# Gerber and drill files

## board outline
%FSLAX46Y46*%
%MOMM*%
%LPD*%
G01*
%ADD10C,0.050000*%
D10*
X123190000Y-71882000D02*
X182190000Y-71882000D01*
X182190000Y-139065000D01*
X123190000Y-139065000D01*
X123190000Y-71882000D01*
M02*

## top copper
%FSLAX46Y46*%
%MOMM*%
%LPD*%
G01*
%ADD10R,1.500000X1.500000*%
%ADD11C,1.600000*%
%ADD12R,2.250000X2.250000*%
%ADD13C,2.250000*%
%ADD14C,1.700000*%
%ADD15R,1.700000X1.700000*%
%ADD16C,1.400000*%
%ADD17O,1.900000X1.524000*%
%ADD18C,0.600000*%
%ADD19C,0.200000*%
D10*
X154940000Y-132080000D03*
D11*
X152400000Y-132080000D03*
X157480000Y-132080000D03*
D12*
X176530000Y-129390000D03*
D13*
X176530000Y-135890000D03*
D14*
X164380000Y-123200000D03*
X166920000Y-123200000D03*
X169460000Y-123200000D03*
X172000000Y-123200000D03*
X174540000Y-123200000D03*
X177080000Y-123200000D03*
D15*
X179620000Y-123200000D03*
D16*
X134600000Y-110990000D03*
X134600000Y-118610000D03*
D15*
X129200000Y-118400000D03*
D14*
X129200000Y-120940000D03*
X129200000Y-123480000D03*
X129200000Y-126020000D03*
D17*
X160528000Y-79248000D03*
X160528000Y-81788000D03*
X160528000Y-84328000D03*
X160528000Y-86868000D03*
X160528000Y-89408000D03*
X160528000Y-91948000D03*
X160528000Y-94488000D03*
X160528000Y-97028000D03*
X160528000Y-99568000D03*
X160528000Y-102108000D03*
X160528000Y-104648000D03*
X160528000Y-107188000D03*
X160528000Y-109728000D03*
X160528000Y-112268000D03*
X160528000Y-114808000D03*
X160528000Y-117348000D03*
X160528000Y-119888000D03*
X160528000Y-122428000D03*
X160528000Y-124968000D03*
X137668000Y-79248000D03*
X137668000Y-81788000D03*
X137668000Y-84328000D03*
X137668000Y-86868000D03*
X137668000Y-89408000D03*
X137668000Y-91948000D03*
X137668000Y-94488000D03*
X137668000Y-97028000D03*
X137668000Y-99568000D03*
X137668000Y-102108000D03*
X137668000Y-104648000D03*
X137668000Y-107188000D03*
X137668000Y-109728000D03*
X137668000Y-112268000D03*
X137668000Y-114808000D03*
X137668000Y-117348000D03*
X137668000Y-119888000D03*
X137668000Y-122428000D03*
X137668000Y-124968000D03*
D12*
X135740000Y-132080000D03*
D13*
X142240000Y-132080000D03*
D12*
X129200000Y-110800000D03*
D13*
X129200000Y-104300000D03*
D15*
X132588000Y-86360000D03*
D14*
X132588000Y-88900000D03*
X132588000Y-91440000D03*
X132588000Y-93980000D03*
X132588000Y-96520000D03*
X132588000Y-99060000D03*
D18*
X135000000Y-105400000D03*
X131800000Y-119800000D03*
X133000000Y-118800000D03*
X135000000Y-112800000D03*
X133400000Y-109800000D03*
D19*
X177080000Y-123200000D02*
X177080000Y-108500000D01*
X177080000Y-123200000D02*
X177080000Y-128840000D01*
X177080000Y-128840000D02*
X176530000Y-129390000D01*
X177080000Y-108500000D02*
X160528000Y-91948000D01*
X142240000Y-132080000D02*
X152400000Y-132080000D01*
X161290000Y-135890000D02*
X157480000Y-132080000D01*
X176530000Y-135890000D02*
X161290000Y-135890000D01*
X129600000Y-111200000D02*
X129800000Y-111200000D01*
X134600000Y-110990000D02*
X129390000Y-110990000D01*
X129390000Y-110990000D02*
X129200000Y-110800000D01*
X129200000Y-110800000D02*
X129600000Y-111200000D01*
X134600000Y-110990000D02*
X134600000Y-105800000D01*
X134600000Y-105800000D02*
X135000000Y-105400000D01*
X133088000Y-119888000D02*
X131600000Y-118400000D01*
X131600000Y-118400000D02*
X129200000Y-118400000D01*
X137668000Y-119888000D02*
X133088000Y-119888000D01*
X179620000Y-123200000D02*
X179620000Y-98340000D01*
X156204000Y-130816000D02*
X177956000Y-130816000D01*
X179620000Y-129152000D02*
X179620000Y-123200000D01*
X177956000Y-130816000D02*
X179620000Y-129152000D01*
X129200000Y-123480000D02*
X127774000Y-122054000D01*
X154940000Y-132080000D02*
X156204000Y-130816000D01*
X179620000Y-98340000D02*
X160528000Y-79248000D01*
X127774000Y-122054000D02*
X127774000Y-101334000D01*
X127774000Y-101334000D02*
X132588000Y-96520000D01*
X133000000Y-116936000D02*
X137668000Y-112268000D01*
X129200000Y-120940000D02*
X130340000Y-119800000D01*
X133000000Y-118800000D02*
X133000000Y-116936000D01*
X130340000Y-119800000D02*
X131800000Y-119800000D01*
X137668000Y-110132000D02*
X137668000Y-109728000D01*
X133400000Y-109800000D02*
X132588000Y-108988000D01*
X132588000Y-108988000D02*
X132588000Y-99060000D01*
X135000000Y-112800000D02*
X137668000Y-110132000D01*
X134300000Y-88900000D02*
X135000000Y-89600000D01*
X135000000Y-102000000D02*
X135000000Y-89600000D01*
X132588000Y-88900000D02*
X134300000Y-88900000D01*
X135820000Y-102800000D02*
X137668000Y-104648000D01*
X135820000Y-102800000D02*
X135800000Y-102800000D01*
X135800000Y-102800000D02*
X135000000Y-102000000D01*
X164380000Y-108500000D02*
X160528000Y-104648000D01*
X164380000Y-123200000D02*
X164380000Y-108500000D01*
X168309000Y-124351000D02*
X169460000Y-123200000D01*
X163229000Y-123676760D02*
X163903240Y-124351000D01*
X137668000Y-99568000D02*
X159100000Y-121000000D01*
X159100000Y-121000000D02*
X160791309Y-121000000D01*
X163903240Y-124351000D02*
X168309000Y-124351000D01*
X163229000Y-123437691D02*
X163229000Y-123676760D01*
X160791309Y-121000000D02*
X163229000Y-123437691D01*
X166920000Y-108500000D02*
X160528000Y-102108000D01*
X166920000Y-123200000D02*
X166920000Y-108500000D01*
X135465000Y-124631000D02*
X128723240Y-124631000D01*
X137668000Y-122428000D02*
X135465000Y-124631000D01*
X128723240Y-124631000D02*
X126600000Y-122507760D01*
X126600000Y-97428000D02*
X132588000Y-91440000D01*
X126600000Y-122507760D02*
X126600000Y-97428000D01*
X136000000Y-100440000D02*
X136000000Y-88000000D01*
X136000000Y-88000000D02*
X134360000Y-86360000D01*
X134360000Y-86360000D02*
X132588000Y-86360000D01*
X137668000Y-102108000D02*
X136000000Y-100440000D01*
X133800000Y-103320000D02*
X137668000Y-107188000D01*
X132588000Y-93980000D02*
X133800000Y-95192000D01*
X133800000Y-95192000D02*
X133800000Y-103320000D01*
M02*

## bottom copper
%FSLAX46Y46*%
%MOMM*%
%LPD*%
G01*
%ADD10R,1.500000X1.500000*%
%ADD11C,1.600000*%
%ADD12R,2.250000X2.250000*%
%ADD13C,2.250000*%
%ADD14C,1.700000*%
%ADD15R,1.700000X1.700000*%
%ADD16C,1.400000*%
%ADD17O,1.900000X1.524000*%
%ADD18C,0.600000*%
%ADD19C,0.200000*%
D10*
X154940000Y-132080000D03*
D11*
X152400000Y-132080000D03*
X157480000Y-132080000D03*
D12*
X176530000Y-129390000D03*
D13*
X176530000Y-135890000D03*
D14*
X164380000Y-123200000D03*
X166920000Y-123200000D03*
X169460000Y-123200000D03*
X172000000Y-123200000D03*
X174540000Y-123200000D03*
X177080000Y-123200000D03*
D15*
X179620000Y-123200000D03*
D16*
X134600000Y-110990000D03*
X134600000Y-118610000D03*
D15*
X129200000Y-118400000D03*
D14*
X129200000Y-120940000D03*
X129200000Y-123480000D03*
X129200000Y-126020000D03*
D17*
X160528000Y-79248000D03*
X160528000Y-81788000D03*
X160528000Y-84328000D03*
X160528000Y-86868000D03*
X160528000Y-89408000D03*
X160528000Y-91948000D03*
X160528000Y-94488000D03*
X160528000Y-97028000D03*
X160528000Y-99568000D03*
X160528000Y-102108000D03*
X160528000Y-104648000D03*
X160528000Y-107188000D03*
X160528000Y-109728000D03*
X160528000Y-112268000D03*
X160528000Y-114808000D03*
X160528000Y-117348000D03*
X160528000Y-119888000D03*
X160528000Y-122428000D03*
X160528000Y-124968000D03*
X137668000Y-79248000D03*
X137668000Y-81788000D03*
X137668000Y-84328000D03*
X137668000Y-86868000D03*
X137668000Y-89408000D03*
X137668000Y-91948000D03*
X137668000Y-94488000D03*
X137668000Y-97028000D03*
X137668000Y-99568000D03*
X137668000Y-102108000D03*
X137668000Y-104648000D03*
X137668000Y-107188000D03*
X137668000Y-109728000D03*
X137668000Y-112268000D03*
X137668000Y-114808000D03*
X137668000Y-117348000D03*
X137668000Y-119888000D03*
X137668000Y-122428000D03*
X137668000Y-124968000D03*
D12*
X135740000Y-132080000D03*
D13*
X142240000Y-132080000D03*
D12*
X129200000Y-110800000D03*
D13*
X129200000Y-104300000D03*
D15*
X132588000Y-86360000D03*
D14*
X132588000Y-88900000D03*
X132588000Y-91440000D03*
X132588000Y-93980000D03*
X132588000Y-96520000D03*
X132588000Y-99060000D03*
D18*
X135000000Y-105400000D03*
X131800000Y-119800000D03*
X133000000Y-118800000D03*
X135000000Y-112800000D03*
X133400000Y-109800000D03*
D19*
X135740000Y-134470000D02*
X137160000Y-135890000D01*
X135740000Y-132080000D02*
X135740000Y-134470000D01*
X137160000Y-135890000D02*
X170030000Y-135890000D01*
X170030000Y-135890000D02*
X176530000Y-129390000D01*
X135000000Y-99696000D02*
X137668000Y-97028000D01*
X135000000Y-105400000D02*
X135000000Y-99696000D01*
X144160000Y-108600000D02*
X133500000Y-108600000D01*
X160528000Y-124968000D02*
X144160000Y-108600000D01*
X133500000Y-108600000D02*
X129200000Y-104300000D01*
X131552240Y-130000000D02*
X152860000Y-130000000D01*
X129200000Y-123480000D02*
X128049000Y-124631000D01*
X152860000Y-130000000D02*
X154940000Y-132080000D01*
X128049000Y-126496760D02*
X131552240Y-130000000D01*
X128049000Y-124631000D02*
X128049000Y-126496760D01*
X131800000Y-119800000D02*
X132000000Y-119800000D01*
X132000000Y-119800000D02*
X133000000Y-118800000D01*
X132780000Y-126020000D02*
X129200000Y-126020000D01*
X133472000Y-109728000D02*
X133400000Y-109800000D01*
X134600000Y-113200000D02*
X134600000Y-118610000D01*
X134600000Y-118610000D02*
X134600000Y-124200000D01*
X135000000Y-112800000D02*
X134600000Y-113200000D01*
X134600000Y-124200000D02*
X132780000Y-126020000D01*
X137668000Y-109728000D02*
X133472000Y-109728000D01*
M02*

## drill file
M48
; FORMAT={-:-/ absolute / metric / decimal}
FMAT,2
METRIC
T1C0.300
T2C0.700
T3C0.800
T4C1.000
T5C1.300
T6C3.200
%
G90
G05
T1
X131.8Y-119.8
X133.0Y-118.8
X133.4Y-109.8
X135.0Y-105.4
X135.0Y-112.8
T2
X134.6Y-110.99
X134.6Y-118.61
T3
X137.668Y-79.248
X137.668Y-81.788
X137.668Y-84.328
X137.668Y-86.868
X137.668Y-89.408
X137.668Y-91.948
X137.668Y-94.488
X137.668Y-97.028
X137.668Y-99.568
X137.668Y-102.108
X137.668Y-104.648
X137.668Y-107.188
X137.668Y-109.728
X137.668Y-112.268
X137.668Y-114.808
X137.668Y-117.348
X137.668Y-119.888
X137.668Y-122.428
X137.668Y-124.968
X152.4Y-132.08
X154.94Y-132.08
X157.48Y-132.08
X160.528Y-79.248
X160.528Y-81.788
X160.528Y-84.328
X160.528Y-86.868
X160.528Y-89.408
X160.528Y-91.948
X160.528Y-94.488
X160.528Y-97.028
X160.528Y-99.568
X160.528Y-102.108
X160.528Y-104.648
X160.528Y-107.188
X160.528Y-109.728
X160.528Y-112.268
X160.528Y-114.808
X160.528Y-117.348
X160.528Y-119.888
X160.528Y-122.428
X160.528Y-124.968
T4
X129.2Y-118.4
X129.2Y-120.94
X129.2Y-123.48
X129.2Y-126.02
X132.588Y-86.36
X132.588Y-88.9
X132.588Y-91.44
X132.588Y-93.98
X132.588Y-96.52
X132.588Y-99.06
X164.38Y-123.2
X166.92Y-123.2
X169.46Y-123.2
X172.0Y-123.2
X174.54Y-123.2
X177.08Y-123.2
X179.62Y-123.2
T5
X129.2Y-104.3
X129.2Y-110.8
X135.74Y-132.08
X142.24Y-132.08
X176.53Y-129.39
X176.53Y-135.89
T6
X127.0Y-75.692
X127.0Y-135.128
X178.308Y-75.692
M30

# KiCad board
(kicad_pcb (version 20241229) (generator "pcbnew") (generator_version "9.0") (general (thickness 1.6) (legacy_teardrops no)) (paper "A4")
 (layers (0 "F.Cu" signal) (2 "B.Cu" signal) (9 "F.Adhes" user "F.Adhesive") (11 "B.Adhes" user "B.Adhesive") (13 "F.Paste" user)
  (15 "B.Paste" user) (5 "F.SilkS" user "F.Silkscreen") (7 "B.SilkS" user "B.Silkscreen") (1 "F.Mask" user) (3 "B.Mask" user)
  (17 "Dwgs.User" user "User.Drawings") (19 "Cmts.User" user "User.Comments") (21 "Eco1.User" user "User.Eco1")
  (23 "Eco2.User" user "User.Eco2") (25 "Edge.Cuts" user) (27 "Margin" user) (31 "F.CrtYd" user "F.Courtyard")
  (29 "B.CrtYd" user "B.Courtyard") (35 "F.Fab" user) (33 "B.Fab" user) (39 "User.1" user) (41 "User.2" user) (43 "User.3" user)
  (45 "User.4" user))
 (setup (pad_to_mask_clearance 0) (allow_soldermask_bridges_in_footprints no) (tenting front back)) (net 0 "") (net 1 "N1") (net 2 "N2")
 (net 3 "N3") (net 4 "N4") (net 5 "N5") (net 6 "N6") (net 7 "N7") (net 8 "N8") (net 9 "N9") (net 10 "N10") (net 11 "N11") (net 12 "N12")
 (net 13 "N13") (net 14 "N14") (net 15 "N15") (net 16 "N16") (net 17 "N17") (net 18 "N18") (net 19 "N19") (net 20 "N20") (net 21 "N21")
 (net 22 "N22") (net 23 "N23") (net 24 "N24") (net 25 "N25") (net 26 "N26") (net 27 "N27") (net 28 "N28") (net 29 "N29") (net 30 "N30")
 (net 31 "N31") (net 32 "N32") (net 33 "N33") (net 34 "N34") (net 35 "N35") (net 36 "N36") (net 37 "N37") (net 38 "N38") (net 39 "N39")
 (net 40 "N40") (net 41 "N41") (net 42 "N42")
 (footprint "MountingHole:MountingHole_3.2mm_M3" (layer "F.Cu") (at 178.308 75.692)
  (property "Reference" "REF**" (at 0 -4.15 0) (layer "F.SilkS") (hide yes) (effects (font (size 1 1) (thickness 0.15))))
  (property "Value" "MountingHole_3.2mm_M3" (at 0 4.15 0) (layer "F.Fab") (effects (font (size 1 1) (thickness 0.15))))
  (pad "" np_thru_hole circle (at 0 0) (size 3.2 3.2) (drill 3.2) (layers "*.Cu" "*.Mask")))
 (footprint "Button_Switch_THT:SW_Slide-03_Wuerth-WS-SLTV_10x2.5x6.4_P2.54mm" (layer "F.Cu") (at 154.94 132.08)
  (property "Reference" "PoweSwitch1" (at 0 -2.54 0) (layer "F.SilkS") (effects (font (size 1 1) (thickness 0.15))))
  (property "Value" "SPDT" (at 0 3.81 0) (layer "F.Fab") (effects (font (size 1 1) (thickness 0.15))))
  (pad "1" thru_hole rect (at 0 0) (size 1.5 1.5) (drill 0.8) (layers "*.Cu" "*.Mask") (remove_unused_layers no) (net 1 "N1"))
  (pad "2" thru_hole circle (at -2.54 0) (size 1.6 1.6) (drill 0.8) (layers "*.Cu" "*.Mask") (remove_unused_layers no) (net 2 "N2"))
  (pad "3" thru_hole circle (at 2.54 0) (size 1.6 1.6) (drill 0.8) (layers "*.Cu" "*.Mask") (remove_unused_layers no) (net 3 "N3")))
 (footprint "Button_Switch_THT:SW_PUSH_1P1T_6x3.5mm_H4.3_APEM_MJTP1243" (layer "F.Cu") (at 176.53 129.39 -90)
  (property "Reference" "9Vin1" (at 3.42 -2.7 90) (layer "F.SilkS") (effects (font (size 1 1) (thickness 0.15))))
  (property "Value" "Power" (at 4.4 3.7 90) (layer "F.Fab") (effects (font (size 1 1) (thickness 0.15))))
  (pad "1" thru_hole rect (at 0 0) (size 2.25 2.25) (drill 1.3) (layers "*.Cu" "*.Mask") (remove_unused_layers no) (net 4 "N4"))
  (pad "2" thru_hole circle (at 6.5 0) (size 2.25 2.25) (drill 1.3) (layers "*.Cu" "*.Mask") (remove_unused_layers no) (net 3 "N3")))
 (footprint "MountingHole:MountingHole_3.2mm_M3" (layer "F.Cu") (at 127 135.128)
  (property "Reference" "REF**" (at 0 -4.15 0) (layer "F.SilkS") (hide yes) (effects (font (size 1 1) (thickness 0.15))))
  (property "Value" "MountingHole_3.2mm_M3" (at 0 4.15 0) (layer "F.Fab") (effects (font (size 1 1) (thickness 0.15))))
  (pad "" np_thru_hole circle (at 0 0) (size 3.2 3.2) (drill 3.2) (layers "*.Cu" "*.Mask")))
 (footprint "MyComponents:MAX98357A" (layer "F.Cu") (at 164.38 123.2 90)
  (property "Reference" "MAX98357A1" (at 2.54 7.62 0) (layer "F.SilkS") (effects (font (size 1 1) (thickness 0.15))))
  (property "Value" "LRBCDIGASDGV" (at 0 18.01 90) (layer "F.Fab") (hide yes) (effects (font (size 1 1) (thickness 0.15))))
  (pad "1" thru_hole circle (at 0 0 270) (size 1.7 1.7) (drill 1) (layers "*.Cu" "*.Mask") (remove_unused_layers no) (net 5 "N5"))
  (pad "2" thru_hole circle (at 0 2.54 270) (size 1.7 1.7) (drill 1) (layers "*.Cu" "*.Mask") (remove_unused_layers no) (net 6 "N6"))
  (pad "3" thru_hole circle (at 0 5.08 270) (size 1.7 1.7) (drill 1) (layers "*.Cu" "*.Mask") (remove_unused_layers no) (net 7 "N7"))
  (pad "4" thru_hole circle (at 0 7.62 270) (size 1.7 1.7) (drill 1) (layers "*.Cu" "*.Mask") (remove_unused_layers no) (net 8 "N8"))
  (pad "5" thru_hole circle (at 0 10.16 270) (size 1.7 1.7) (drill 1) (layers "*.Cu" "*.Mask") (remove_unused_layers no) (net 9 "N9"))
  (pad "6" thru_hole circle (at 0 12.7 270) (size 1.7 1.7) (drill 1) (layers "*.Cu" "*.Mask") (remove_unused_layers no) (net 4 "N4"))
  (pad "7" thru_hole rect (at 0 15.24 270) (size 1.7 1.7) (drill 1) (layers "*.Cu" "*.Mask") (remove_unused_layers no) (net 1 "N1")))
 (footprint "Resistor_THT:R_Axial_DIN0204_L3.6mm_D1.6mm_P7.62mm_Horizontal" (layer "F.Cu") (at 134.6 110.99 -90)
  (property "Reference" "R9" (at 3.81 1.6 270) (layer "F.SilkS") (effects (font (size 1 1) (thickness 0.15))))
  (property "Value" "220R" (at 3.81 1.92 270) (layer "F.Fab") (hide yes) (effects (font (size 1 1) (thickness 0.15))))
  (pad "1" thru_hole circle (at 0 0 270) (size 1.4 1.4) (drill 0.7) (layers "*.Cu" "*.Mask") (remove_unused_layers no) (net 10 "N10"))
  (pad "2" thru_hole circle (at 7.62 0 270) (size 1.4 1.4) (drill 0.7) (layers "*.Cu" "*.Mask") (remove_unused_layers no) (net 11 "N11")))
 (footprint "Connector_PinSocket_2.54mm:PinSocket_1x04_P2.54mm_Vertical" (layer "F.Cu") (at 129.2 118.4)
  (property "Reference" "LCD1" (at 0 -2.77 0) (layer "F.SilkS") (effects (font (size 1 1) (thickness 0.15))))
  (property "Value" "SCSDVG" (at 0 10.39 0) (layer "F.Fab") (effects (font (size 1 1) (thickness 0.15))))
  (pad "1" thru_hole rect (at 0 0) (size 1.7 1.7) (drill 1) (layers "*.Cu" "*.Mask") (remove_unused_layers no) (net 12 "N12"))
  (pad "2" thru_hole circle (at 0 2.54) (size 1.7 1.7) (drill 1) (layers "*.Cu" "*.Mask") (remove_unused_layers no) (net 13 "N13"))
  (pad "3" thru_hole circle (at 0 5.08) (size 1.7 1.7) (drill 1) (layers "*.Cu" "*.Mask") (remove_unused_layers no) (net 1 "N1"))
  (pad "4" thru_hole circle (at 0 7.62) (size 1.7 1.7) (drill 1) (layers "*.Cu" "*.Mask") (remove_unused_layers no) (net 11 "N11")))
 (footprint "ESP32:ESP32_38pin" (layer "F.Cu") (at 148.984183 102.273111 180)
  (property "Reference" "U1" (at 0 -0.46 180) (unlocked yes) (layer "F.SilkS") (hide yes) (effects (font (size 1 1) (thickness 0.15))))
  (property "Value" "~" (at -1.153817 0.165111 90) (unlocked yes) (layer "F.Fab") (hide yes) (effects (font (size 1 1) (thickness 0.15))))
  (pad "1" thru_hole oval (at -11.543817 23.025111 90) (size 1.524 1.9) (drill 0.8) (layers "*.Cu" "*.Mask") (remove_unused_layers no)
   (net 1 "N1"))
  (pad "2" thru_hole oval (at -11.543817 20.485111 90) (size 1.524 1.9) (drill 0.8) (layers "*.Cu" "*.Mask") (remove_unused_layers no)
   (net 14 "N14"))
  (pad "3" thru_hole oval (at -11.543817 17.945111 90) (size 1.524 1.9) (drill 0.8) (layers "*.Cu" "*.Mask") (remove_unused_layers no)
   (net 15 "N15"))
  (pad "4" thru_hole oval (at -11.543817 15.405111 90) (size 1.524 1.9) (drill 0.8) (layers "*.Cu" "*.Mask") (remove_unused_layers no)
   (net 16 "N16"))
  (pad "5" thru_hole oval (at -11.543817 12.865111 90) (size 1.524 1.9) (drill 0.8) (layers "*.Cu" "*.Mask") (remove_unused_layers no)
   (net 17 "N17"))
  (pad "6" thru_hole oval (at -11.543817 10.325111 90) (size 1.524 1.9) (drill 0.8) (layers "*.Cu" "*.Mask") (remove_unused_layers no)
   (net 4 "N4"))
  (pad "7" thru_hole oval (at -11.543817 7.785111 90) (size 1.524 1.9) (drill 0.8) (layers "*.Cu" "*.Mask") (remove_unused_layers no)
   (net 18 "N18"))
  (pad "8" thru_hole oval (at -11.543817 5.245111 90) (size 1.524 1.9) (drill 0.8) (layers "*.Cu" "*.Mask") (remove_unused_layers no)
   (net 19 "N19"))
  (pad "9" thru_hole oval (at -11.543817 2.705111 90) (size 1.524 1.9) (drill 0.8) (layers "*.Cu" "*.Mask") (remove_unused_layers no)
   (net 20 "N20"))
  (pad "10" thru_hole oval (at -11.543817 0.165111 90) (size 1.524 1.9) (drill 0.8) (layers "*.Cu" "*.Mask") (remove_unused_layers no)
   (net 6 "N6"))
  (pad "11" thru_hole oval (at -11.543817 -2.374889 90) (size 1.524 1.9) (drill 0.8) (layers "*.Cu" "*.Mask") (remove_unused_layers no)
   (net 5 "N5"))
  (pad "12" thru_hole oval (at -11.543817 -4.914889 90) (size 1.524 1.9) (drill 0.8) (layers "*.Cu" "*.Mask") (remove_unused_layers no)
   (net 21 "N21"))
  (pad "13" thru_hole oval (at -11.543817 -7.454889 90) (size 1.524 1.9) (drill 0.8) (layers "*.Cu" "*.Mask") (remove_unused_layers no)
   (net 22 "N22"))
  (pad "14" thru_hole oval (at -11.543817 -9.994889 90) (size 1.524 1.9) (drill 0.8) (layers "*.Cu" "*.Mask") (remove_unused_layers no)
   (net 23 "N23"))
  (pad "15" thru_hole oval (at -11.543817 -12.534889 90) (size 1.524 1.9) (drill 0.8) (layers "*.Cu" "*.Mask") (remove_unused_layers no)
   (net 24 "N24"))
  (pad "16" thru_hole oval (at -11.543817 -15.074889 90) (size 1.524 1.9) (drill 0.8) (layers "*.Cu" "*.Mask") (remove_unused_layers no)
   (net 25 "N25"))
  (pad "17" thru_hole oval (at -11.543817 -17.614889 90) (size 1.524 1.9) (drill 0.8) (layers "*.Cu" "*.Mask") (remove_unused_layers no)
   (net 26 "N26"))
  (pad "18" thru_hole oval (at -11.543817 -20.154889 90) (size 1.524 1.9) (drill 0.8) (layers "*.Cu" "*.Mask") (remove_unused_layers no)
   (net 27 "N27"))
  (pad "19" thru_hole oval (at -11.543817 -22.694889 90) (size 1.524 1.9) (drill 0.8) (layers "*.Cu" "*.Mask") (remove_unused_layers no)
   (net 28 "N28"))
  (pad "20" thru_hole oval (at 11.316183 23.025111 90) (size 1.524 1.9) (drill 0.8) (layers "*.Cu" "*.Mask") (remove_unused_layers no)
   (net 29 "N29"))
  (pad "21" thru_hole oval (at 11.316183 20.485111 90) (size 1.524 1.9) (drill 0.8) (layers "*.Cu" "*.Mask") (remove_unused_layers no)
   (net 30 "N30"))
  (pad "22" thru_hole oval (at 11.316183 17.945111 90) (size 1.524 1.9) (drill 0.8) (layers "*.Cu" "*.Mask") (remove_unused_layers no)
   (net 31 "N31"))
  (pad "23" thru_hole oval (at 11.316183 15.405111 90) (size 1.524 1.9) (drill 0.8) (layers "*.Cu" "*.Mask") (remove_unused_layers no)
   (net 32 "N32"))
  (pad "24" thru_hole oval (at 11.316183 12.865111 90) (size 1.524 1.9) (drill 0.8) (layers "*.Cu" "*.Mask") (remove_unused_layers no)
   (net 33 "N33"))
  (pad "25" thru_hole oval (at 11.316183 10.325111 90) (size 1.524 1.9) (drill 0.8) (layers "*.Cu" "*.Mask") (remove_unused_layers no)
   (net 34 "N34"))
  (pad "26" thru_hole oval (at 11.316183 7.785111 90) (size 1.524 1.9) (drill 0.8) (layers "*.Cu" "*.Mask") (remove_unused_layers no)
   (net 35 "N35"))
  (pad "27" thru_hole oval (at 11.316183 5.245111 90) (size 1.524 1.9) (drill 0.8) (layers "*.Cu" "*.Mask") (remove_unused_layers no)
   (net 10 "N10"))
  (pad "28" thru_hole oval (at 11.316183 2.705111 90) (size 1.524 1.9) (drill 0.8) (layers "*.Cu" "*.Mask") (remove_unused_layers no)
   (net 7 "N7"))
  (pad "29" thru_hole oval (at 11.316183 0.165111 90) (size 1.524 1.9) (drill 0.8) (layers "*.Cu" "*.Mask") (remove_unused_layers no)
   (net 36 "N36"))
  (pad "30" thru_hole oval (at 11.316183 -2.374889 90) (size 1.524 1.9) (drill 0.8) (layers "*.Cu" "*.Mask") (remove_unused_layers no)
   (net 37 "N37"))
  (pad "31" thru_hole oval (at 11.316183 -4.914889 90) (size 1.524 1.9) (drill 0.8) (layers "*.Cu" "*.Mask") (remove_unused_layers no)
   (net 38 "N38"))
  (pad "32" thru_hole oval (at 11.316183 -7.454889 90) (size 1.524 1.9) (drill 0.8) (layers "*.Cu" "*.Mask") (remove_unused_layers no)
   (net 11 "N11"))
  (pad "33" thru_hole oval (at 11.316183 -9.994889 90) (size 1.524 1.9) (drill 0.8) (layers "*.Cu" "*.Mask") (remove_unused_layers no)
   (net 13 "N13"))
  (pad "34" thru_hole oval (at 11.316183 -12.534889 90) (size 1.524 1.9) (drill 0.8) (layers "*.Cu" "*.Mask") (remove_unused_layers no)
   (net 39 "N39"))
  (pad "35" thru_hole oval (at 11.316183 -15.074889 90) (size 1.524 1.9) (drill 0.8) (layers "*.Cu" "*.Mask") (remove_unused_layers no)
   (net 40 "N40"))
  (pad "36" thru_hole oval (at 11.316183 -17.614889 90) (size 1.524 1.9) (drill 0.8) (layers "*.Cu" "*.Mask") (remove_unused_layers no)
   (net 12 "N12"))
  (pad "37" thru_hole oval (at 11.316183 -20.154889 90) (size 1.524 1.9) (drill 0.8) (layers "*.Cu" "*.Mask") (remove_unused_layers no)
   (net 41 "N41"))
  (pad "38" thru_hole oval (at 11.316183 -22.694889 90) (size 1.524 1.9) (drill 0.8) (layers "*.Cu" "*.Mask") (remove_unused_layers no)
   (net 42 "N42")))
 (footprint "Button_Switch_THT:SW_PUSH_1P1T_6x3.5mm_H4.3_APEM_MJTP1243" (layer "F.Cu") (at 135.74 132.08)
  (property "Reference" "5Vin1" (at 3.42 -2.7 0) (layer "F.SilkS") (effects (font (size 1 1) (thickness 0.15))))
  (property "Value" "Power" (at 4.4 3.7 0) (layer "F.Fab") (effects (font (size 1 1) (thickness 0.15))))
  (pad "1" thru_hole rect (at 0 0 90) (size 2.25 2.25) (drill 1.3) (layers "*.Cu" "*.Mask") (remove_unused_layers no) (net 4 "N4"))
  (pad "2" thru_hole circle (at 6.5 0 90) (size 2.25 2.25) (drill 1.3) (layers "*.Cu" "*.Mask") (remove_unused_layers no) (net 2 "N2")))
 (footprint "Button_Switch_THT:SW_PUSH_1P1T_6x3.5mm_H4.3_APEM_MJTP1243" (layer "F.Cu") (at 129.2 110.8 90)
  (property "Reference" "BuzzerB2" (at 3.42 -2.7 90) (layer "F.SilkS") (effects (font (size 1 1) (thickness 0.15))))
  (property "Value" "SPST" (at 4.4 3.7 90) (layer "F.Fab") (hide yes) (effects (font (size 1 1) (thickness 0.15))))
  (pad "1" thru_hole rect (at 0 0 180) (size 2.25 2.25) (drill 1.3) (layers "*.Cu" "*.Mask") (remove_unused_layers no) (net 10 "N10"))
  (pad "2" thru_hole circle (at 6.5 0 180) (size 2.25 2.25) (drill 1.3) (layers "*.Cu" "*.Mask") (remove_unused_layers no) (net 28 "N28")))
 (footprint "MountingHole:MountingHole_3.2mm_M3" (layer "F.Cu") (at 127 75.692)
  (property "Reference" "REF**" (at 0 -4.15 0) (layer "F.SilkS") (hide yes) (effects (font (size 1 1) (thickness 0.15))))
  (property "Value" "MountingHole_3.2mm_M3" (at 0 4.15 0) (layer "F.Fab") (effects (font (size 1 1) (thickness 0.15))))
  (pad "" np_thru_hole circle (at 0 0) (size 3.2 3.2) (drill 3.2) (layers "*.Cu" "*.Mask")))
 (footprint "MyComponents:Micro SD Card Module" (layer "B.Cu") (at 132.588 86.435 180)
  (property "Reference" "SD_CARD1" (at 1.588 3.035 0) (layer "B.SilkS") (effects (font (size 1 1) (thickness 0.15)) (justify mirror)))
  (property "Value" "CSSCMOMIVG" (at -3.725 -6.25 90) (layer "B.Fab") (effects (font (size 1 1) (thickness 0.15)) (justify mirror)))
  (pad "1" thru_hole rect (at 0 0.075 180) (size 1.7 1.7) (drill 1) (layers "*.Cu" "*.Mask") (remove_unused_layers no) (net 36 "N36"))
  (pad "2" thru_hole circle (at 0 -2.465 180) (size 1.7 1.7) (drill 1) (layers "*.Cu" "*.Mask") (remove_unused_layers no) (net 37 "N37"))
  (pad "3" thru_hole circle (at 0 -5.005 180) (size 1.7 1.7) (drill 1) (layers "*.Cu" "*.Mask") (remove_unused_layers no) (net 41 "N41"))
  (pad "4" thru_hole circle (at 0 -7.545 180) (size 1.7 1.7) (drill 1) (layers "*.Cu" "*.Mask") (remove_unused_layers no) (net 38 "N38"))
  (pad "5" thru_hole circle (at 0 -10.085 180) (size 1.7 1.7) (drill 1) (layers "*.Cu" "*.Mask") (remove_unused_layers no) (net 1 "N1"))
  (pad "6" thru_hole circle (at 0 -12.625 180) (size 1.7 1.7) (drill 1) (layers "*.Cu" "*.Mask") (remove_unused_layers no) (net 11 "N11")))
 (gr_rect (start 123.19 71.882) (end 182.19 139.065) (stroke (width 0.05) (type solid)) (fill no) (layer "Edge.Cuts"))
 (segment (start 177.08 123.2) (end 177.08 108.5) (width 0.2) (layer "F.Cu") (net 4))
 (segment (start 177.08 123.2) (end 177.08 128.84) (width 0.2) (layer "F.Cu") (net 4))
 (segment (start 177.08 128.84) (end 176.53 129.39) (width 0.2) (layer "F.Cu") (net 4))
 (segment (start 177.08 108.5) (end 160.528 91.948) (width 0.2) (layer "F.Cu") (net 4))
 (segment (start 135.74 134.47) (end 137.16 135.89) (width 0.2) (layer "B.Cu") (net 4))
 (segment (start 135.74 132.08) (end 135.74 134.47) (width 0.2) (layer "B.Cu") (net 4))
 (segment (start 137.16 135.89) (end 170.03 135.89) (width 0.2) (layer "B.Cu") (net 4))
 (segment (start 170.03 135.89) (end 176.53 129.39) (width 0.2) (layer "B.Cu") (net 4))
 (segment (start 142.24 132.08) (end 152.4 132.08) (width 0.2) (layer "F.Cu") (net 2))
 (segment (start 161.29 135.89) (end 157.48 132.08) (width 0.2) (layer "F.Cu") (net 3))
 (segment (start 176.53 135.89) (end 161.29 135.89) (width 0.2) (layer "F.Cu") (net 3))
 (segment (start 129.6 111.2) (end 129.8 111.2) (width 0.2) (layer "F.Cu") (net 10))
 (segment (start 134.6 110.99) (end 129.39 110.99) (width 0.2) (layer "F.Cu") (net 10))
 (segment (start 129.39 110.99) (end 129.2 110.8) (width 0.2) (layer "F.Cu") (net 10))
 (segment (start 129.2 110.8) (end 129.6 111.2) (width 0.2) (layer "F.Cu") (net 10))
 (segment (start 134.6 110.99) (end 134.6 105.8) (width 0.2) (layer "F.Cu") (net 10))
 (segment (start 134.6 105.8) (end 135 105.4) (width 0.2) (layer "F.Cu") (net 10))
 (via (at 135 105.4) (size 0.6) (drill 0.3) (layers "F.Cu" "B.Cu") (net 10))
 (segment (start 135 99.696) (end 137.668 97.028) (width 0.2) (layer "B.Cu") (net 10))
 (segment (start 135 105.4) (end 135 99.696) (width 0.2) (layer "B.Cu") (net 10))
 (segment (start 144.16 108.6) (end 133.5 108.6) (width 0.2) (layer "B.Cu") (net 28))
 (segment (start 160.528 124.968) (end 144.16 108.6) (width 0.2) (layer "B.Cu") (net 28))
 (segment (start 133.5 108.6) (end 129.2 104.3) (width 0.2) (layer "B.Cu") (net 28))
 (segment (start 133.088 119.888) (end 131.6 118.4) (width 0.2) (layer "F.Cu") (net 12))
 (segment (start 131.6 118.4) (end 129.2 118.4) (width 0.2) (layer "F.Cu") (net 12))
 (segment (start 137.668 119.888) (end 133.088 119.888) (width 0.2) (layer "F.Cu") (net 12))
 (segment (start 179.62 123.2) (end 179.62 98.34) (width 0.2) (layer "F.Cu") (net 1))
 (segment (start 156.204 130.816) (end 177.956 130.816) (width 0.2) (layer "F.Cu") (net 1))
 (segment (start 179.62 129.152) (end 179.62 123.2) (width 0.2) (layer "F.Cu") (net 1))
 (segment (start 177.956 130.816) (end 179.62 129.152) (width 0.2) (layer "F.Cu") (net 1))
 (segment (start 129.2 123.48) (end 127.774 122.054) (width 0.2) (layer "F.Cu") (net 1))
 (segment (start 154.94 132.08) (end 156.204 130.816) (width 0.2) (layer "F.Cu") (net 1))
 (segment (start 179.62 98.34) (end 160.528 79.248) (width 0.2) (layer "F.Cu") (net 1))
 (segment (start 127.774 122.054) (end 127.774 101.334) (width 0.2) (layer "F.Cu") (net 1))
 (segment (start 127.774 101.334) (end 132.588 96.52) (width 0.2) (layer "F.Cu") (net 1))
 (segment (start 131.55224 130) (end 152.86 130) (width 0.2) (layer "B.Cu") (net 1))
 (segment (start 129.2 123.48) (end 128.049 124.631) (width 0.2) (layer "B.Cu") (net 1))
 (segment (start 152.86 130) (end 154.94 132.08) (width 0.2) (layer "B.Cu") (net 1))
 (segment (start 128.049 126.49676) (end 131.55224 130) (width 0.2) (layer "B.Cu") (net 1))
 (segment (start 128.049 124.631) (end 128.049 126.49676) (width 0.2) (layer "B.Cu") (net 1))
 (segment (start 133 116.936) (end 137.668 112.268) (width 0.2) (layer "F.Cu") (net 13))
 (segment (start 129.2 120.94) (end 130.34 119.8) (width 0.2) (layer "F.Cu") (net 13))
 (segment (start 133 118.8) (end 133 116.936) (width 0.2) (layer "F.Cu") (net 13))
 (segment (start 130.34 119.8) (end 131.8 119.8) (width 0.2) (layer "F.Cu") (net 13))
 (via (at 131.8 119.8) (size 0.6) (drill 0.3) (layers "F.Cu" "B.Cu") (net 13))
 (via (at 133 118.8) (size 0.6) (drill 0.3) (layers "F.Cu" "B.Cu") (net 13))
 (segment (start 131.8 119.8) (end 132 119.8) (width 0.2) (layer "B.Cu") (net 13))
 (segment (start 132 119.8) (end 133 118.8) (width 0.2) (layer "B.Cu") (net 13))
 (segment (start 137.668 110.132) (end 137.668 109.728) (width 0.2) (layer "F.Cu") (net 11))
 (segment (start 133.4 109.8) (end 132.588 108.988) (width 0.2) (layer "F.Cu") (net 11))
 (segment (start 132.588 108.988) (end 132.588 99.06) (width 0.2) (layer "F.Cu") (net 11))
 (segment (start 135 112.8) (end 137.668 110.132) (width 0.2) (layer "F.Cu") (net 11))
 (via (at 135 112.8) (size 0.6) (drill 0.3) (layers "F.Cu" "B.Cu") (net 11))
 (via (at 133.4 109.8) (size 0.6) (drill 0.3) (layers "F.Cu" "B.Cu") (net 11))
 (segment (start 132.78 126.02) (end 129.2 126.02) (width 0.2) (layer "B.Cu") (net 11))
 (segment (start 133.472 109.728) (end 133.4 109.8) (width 0.2) (layer "B.Cu") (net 11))
 (segment (start 134.6 113.2) (end 134.6 118.61) (width 0.2) (layer "B.Cu") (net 11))
 (segment (start 134.6 118.61) (end 134.6 124.2) (width 0.2) (layer "B.Cu") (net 11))
 (segment (start 135 112.8) (end 134.6 113.2) (width 0.2) (layer "B.Cu") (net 11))
 (segment (start 134.6 124.2) (end 132.78 126.02) (width 0.2) (layer "B.Cu") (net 11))
 (segment (start 137.668 109.728) (end 133.472 109.728) (width 0.2) (layer "B.Cu") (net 11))
 (segment (start 134.3 88.9) (end 135 89.6) (width 0.2) (layer "F.Cu") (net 37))
 (segment (start 135 102) (end 135 89.6) (width 0.2) (layer "F.Cu") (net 37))
 (segment (start 132.588 88.9) (end 134.3 88.9) (width 0.2) (layer "F.Cu") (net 37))
 (segment (start 135.82 102.8) (end 137.668 104.648) (width 0.2) (layer "F.Cu") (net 37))
 (segment (start 135.82 102.8) (end 135.8 102.8) (width 0.2) (layer "F.Cu") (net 37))
 (segment (start 135.8 102.8) (end 135 102) (width 0.2) (layer "F.Cu") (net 37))
 (segment (start 164.38 108.5) (end 160.528 104.648) (width 0.2) (layer "F.Cu") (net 5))
 (segment (start 164.38 123.2) (end 164.38 108.5) (width 0.2) (layer "F.Cu") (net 5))
 (segment (start 168.309 124.351) (end 169.46 123.2) (width 0.2) (layer "F.Cu") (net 7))
 (segment (start 163.229 123.67676) (end 163.90324 124.351) (width 0.2) (layer "F.Cu") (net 7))
 (segment (start 137.668 99.568) (end 159.1 121) (width 0.2) (layer "F.Cu") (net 7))
 (segment (start 159.1 121) (end 160.791309 121) (width 0.2) (layer "F.Cu") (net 7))
 (segment (start 163.90324 124.351) (end 168.309 124.351) (width 0.2) (layer "F.Cu") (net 7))
 (segment (start 163.229 123.437691) (end 163.229 123.67676) (width 0.2) (layer "F.Cu") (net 7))
 (segment (start 160.791309 121) (end 163.229 123.437691) (width 0.2) (layer "F.Cu") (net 7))
 (segment (start 166.92 108.5) (end 160.528 102.108) (width 0.2) (layer "F.Cu") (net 6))
 (segment (start 166.92 123.2) (end 166.92 108.5) (width 0.2) (layer "F.Cu") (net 6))
 (segment (start 135.465 124.631) (end 128.72324 124.631) (width 0.2) (layer "F.Cu") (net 41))
 (segment (start 137.668 122.428) (end 135.465 124.631) (width 0.2) (layer "F.Cu") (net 41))
 (segment (start 128.72324 124.631) (end 126.6 122.50776) (width 0.2) (layer "F.Cu") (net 41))
 (segment (start 126.6 97.428) (end 132.588 91.44) (width 0.2) (layer "F.Cu") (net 41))
 (segment (start 126.6 122.50776) (end 126.6 97.428) (width 0.2) (layer "F.Cu") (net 41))
 (segment (start 136 100.44) (end 136 88) (width 0.2) (layer "F.Cu") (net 36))
 (segment (start 136 88) (end 134.36 86.36) (width 0.2) (layer "F.Cu") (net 36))
 (segment (start 134.36 86.36) (end 132.588 86.36) (width 0.2) (layer "F.Cu") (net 36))
 (segment (start 137.668 102.108) (end 136 100.44) (width 0.2) (layer "F.Cu") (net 36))
 (segment (start 133.8 103.32) (end 137.668 107.188) (width 0.2) (layer "F.Cu") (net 38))
 (segment (start 132.588 93.98) (end 133.8 95.192) (width 0.2) (layer "F.Cu") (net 38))
 (segment (start 133.8 95.192) (end 133.8 103.32) (width 0.2) (layer "F.Cu") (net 38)))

